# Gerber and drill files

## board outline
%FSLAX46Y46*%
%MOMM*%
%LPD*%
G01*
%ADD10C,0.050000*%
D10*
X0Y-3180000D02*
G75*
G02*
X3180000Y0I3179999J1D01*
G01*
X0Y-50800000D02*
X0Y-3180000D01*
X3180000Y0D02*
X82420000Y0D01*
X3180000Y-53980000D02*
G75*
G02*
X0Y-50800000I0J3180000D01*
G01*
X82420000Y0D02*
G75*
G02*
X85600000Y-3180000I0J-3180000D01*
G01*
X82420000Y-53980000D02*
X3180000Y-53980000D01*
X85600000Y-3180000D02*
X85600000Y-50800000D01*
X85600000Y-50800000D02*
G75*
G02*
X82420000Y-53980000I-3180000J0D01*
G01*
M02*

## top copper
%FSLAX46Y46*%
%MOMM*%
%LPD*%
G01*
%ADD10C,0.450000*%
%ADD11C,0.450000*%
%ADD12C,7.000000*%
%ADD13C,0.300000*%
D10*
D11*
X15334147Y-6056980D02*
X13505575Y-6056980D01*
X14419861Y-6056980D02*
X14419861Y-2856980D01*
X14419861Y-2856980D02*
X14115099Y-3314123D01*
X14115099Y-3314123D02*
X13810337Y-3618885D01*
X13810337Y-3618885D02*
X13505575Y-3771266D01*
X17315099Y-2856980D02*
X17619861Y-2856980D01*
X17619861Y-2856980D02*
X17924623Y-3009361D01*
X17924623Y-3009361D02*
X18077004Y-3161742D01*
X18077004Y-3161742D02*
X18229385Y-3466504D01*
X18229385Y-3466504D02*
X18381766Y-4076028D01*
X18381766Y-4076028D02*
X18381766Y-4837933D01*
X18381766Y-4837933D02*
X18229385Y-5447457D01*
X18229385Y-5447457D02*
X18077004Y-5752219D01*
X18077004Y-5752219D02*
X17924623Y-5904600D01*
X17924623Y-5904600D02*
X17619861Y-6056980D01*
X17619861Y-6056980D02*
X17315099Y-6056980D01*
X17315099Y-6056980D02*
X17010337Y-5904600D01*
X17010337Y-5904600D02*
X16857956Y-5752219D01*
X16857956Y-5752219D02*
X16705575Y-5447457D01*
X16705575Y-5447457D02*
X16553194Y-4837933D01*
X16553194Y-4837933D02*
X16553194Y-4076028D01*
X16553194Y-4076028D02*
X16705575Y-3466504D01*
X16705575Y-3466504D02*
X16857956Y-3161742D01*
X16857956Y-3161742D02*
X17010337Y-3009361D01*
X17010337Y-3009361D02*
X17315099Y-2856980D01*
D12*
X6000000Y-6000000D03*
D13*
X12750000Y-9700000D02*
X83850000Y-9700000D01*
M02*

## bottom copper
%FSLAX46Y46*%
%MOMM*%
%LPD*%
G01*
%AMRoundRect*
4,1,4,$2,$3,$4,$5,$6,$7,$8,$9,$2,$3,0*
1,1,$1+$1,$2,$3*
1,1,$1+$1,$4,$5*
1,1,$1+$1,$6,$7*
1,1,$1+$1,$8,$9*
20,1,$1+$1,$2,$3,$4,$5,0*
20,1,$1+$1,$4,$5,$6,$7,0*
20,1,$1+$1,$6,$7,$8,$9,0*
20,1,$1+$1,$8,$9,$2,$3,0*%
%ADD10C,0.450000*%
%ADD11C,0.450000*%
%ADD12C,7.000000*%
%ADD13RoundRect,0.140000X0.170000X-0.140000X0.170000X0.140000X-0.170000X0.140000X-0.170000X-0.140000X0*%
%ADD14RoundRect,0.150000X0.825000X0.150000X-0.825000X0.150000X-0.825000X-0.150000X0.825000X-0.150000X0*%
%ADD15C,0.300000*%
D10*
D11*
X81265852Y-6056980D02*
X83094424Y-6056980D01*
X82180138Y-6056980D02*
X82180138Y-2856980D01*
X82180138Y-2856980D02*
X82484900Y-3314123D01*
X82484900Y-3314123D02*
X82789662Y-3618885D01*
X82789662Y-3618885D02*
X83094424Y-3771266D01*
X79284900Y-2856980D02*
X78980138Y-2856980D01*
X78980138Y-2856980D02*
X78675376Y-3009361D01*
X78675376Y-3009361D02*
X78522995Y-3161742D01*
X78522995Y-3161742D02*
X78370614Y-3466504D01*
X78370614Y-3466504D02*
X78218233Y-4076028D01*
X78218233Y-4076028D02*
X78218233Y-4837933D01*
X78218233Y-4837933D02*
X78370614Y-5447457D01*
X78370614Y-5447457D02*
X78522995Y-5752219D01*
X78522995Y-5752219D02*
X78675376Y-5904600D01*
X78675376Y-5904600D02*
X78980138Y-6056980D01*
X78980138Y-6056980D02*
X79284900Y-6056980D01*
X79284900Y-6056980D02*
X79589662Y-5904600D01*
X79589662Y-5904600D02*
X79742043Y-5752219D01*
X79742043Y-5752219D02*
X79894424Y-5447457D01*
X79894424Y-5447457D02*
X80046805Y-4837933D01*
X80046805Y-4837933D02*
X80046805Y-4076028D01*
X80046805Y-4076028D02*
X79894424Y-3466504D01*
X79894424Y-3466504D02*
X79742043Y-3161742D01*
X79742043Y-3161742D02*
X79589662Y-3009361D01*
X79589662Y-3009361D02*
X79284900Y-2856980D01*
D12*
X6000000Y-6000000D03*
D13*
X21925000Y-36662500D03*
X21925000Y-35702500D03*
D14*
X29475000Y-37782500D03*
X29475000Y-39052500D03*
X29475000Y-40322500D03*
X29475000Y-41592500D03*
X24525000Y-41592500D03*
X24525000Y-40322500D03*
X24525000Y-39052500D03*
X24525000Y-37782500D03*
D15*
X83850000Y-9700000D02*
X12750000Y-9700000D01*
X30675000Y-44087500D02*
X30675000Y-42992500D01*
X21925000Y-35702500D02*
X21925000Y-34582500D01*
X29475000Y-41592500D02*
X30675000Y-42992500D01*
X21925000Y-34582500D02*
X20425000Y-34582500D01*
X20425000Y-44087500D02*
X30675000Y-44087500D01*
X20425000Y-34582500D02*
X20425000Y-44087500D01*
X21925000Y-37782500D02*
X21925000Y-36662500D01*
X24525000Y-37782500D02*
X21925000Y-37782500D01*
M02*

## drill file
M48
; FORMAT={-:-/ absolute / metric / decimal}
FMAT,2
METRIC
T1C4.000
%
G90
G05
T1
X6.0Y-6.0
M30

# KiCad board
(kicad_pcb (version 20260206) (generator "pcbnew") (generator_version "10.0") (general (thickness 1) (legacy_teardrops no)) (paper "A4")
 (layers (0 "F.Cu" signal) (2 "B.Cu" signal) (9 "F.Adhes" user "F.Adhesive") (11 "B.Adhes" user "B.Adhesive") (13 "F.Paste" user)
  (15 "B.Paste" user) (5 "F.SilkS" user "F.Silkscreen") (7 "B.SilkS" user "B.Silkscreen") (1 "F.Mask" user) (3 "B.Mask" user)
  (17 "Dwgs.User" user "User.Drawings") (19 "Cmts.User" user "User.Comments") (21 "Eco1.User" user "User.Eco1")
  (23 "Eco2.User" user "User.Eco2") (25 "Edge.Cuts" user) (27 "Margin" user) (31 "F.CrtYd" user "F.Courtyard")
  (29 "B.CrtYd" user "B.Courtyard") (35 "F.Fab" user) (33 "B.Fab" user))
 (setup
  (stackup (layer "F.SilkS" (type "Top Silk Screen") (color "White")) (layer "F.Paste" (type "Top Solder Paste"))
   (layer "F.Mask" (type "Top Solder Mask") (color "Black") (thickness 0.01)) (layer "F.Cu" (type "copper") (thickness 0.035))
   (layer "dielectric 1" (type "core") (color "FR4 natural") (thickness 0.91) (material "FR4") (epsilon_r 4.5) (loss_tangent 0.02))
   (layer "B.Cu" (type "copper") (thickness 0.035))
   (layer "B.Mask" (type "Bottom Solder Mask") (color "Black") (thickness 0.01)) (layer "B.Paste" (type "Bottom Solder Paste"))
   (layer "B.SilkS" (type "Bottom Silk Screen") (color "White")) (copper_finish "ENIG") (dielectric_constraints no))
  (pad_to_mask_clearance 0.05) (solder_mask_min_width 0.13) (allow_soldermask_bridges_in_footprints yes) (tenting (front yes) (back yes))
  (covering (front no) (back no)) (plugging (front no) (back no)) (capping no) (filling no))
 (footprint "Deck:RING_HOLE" (layer "F.Cu") (at 6 6)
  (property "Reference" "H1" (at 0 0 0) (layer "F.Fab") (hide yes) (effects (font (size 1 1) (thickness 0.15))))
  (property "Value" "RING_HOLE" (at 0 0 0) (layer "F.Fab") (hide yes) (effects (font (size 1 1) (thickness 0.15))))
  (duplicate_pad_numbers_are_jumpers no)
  (pad "" thru_hole circle (at 0 0) (size 7 7) (drill 4) (layers "*.Cu" "*.Mask") (remove_unused_layers no)))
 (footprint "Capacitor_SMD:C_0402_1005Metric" (layer "B.Cu") (at 21.925 36.1825 90)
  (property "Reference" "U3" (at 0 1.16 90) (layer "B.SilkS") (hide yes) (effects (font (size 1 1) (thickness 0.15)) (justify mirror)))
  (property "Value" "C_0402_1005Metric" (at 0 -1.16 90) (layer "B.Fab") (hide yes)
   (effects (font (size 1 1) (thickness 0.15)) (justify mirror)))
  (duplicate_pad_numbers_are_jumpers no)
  (pad "1" smd roundrect (at -0.48 0 90) (size 0.56 0.62) (layers "B.Cu" "B.Mask") (roundrect_rratio 0.25) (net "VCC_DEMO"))
  (pad "2" smd roundrect (at 0.48 0 90) (size 0.56 0.62) (layers "B.Cu" "B.Mask") (roundrect_rratio 0.25) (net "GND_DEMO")))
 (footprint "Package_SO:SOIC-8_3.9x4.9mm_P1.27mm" (layer "B.Cu") (at 27 39.6875 180)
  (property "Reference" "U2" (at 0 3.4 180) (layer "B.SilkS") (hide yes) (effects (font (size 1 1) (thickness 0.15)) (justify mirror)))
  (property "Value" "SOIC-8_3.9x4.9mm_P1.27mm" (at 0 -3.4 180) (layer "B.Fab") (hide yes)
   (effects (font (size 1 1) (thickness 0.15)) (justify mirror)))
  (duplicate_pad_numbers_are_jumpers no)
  (pad "1" smd roundrect (at -2.475 1.905 180) (size 1.95 0.6) (layers "B.Cu" "B.Mask") (roundrect_rratio 0.25))
  (pad "2" smd roundrect (at -2.475 0.635 180) (size 1.95 0.6) (layers "B.Cu" "B.Mask") (roundrect_rratio 0.25))
  (pad "3" smd roundrect (at -2.475 -0.635 180) (size 1.95 0.6) (layers "B.Cu" "B.Mask") (roundrect_rratio 0.25))
  (pad "4" smd roundrect (at -2.475 -1.905 180) (size 1.95 0.6) (layers "B.Cu" "B.Mask") (roundrect_rratio 0.25) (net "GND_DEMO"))
  (pad "5" smd roundrect (at 2.475 -1.905 180) (size 1.95 0.6) (layers "B.Cu" "B.Mask") (roundrect_rratio 0.25))
  (pad "6" smd roundrect (at 2.475 -0.635 180) (size 1.95 0.6) (layers "B.Cu" "B.Mask") (roundrect_rratio 0.25))
  (pad "7" smd roundrect (at 2.475 0.635 180) (size 1.95 0.6) (layers "B.Cu" "B.Mask") (roundrect_rratio 0.25))
  (pad "8" smd roundrect (at 2.475 1.905 180) (size 1.95 0.6) (layers "B.Cu" "B.Mask") (roundrect_rratio 0.25) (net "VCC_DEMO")))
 (gr_arc (start 0 3.18) (mid 0.9314 0.9314) (end 3.18 0) (stroke (width 0.05) (type solid)) (layer "Edge.Cuts"))
 (gr_line (start 0 50.8) (end 0 3.18) (stroke (width 0.05) (type solid)) (layer "Edge.Cuts"))
 (gr_line (start 3.18 0) (end 82.42 0) (stroke (width 0.05) (type solid)) (layer "Edge.Cuts"))
 (gr_arc (start 3.18 53.98) (mid 0.9314 53.0486) (end 0 50.8) (stroke (width 0.05) (type solid)) (layer "Edge.Cuts"))
 (gr_arc (start 82.42 0) (mid 84.6686 0.9314) (end 85.6 3.18) (stroke (width 0.05) (type solid)) (layer "Edge.Cuts"))
 (gr_line (start 82.42 53.98) (end 3.18 53.98) (stroke (width 0.05) (type solid)) (layer "Edge.Cuts"))
 (gr_line (start 85.6 3.18) (end 85.6 50.8) (stroke (width 0.05) (type solid)) (layer "Edge.Cuts"))
 (gr_arc (start 85.6 50.8) (mid 84.6686 53.0486) (end 82.42 53.98) (stroke (width 0.05) (type solid)) (layer "Edge.Cuts"))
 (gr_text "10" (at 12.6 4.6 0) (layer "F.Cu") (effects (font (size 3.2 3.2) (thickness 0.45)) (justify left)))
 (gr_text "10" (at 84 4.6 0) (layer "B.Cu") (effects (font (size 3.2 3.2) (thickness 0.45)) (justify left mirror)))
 (segment (start 12.75 9.7) (end 83.85 9.7) (width 0.3) (layer "F.Cu") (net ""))
 (segment (start 83.85 9.7) (end 12.75 9.7) (width 0.3) (layer "B.Cu") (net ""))
 (segment (start 30.675 44.0875) (end 30.675 42.9925) (width 0.3) (layer "B.Cu") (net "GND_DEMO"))
 (segment (start 21.925 35.7025) (end 21.925 34.5825) (width 0.3) (layer "B.Cu") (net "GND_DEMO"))
 (segment (start 29.475 41.5925) (end 30.675 42.9925) (width 0.3) (layer "B.Cu") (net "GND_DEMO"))
 (segment (start 21.925 34.5825) (end 20.425 34.5825) (width 0.3) (layer "B.Cu") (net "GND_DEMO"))
 (segment (start 20.425 44.0875) (end 30.675 44.0875) (width 0.3) (layer "B.Cu") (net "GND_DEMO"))
 (segment (start 20.425 34.5825) (end 20.425 44.0875) (width 0.3) (layer "B.Cu") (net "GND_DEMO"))
 (segment (start 21.925 37.7825) (end 21.925 36.6625) (width 0.3) (layer "B.Cu") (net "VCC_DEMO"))
 (segment (start 24.525 37.7825) (end 21.925 37.7825) (width 0.3) (layer "B.Cu") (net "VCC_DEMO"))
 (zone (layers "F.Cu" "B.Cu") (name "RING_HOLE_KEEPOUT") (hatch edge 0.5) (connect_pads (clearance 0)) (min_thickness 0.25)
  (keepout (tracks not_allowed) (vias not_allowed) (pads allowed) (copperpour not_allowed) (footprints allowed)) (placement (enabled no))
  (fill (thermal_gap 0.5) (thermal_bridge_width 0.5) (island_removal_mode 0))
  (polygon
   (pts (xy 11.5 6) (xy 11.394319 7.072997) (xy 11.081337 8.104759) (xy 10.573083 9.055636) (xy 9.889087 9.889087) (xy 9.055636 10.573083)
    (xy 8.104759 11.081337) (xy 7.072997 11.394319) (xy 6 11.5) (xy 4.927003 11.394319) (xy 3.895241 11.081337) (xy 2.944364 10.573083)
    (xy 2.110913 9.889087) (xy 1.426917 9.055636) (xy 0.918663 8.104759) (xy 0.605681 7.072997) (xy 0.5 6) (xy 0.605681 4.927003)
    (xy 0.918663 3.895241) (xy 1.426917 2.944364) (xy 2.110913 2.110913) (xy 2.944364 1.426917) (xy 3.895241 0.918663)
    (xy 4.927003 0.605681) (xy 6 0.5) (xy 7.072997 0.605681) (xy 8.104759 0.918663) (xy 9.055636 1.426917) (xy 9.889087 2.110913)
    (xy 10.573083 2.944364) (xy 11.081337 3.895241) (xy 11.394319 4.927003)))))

